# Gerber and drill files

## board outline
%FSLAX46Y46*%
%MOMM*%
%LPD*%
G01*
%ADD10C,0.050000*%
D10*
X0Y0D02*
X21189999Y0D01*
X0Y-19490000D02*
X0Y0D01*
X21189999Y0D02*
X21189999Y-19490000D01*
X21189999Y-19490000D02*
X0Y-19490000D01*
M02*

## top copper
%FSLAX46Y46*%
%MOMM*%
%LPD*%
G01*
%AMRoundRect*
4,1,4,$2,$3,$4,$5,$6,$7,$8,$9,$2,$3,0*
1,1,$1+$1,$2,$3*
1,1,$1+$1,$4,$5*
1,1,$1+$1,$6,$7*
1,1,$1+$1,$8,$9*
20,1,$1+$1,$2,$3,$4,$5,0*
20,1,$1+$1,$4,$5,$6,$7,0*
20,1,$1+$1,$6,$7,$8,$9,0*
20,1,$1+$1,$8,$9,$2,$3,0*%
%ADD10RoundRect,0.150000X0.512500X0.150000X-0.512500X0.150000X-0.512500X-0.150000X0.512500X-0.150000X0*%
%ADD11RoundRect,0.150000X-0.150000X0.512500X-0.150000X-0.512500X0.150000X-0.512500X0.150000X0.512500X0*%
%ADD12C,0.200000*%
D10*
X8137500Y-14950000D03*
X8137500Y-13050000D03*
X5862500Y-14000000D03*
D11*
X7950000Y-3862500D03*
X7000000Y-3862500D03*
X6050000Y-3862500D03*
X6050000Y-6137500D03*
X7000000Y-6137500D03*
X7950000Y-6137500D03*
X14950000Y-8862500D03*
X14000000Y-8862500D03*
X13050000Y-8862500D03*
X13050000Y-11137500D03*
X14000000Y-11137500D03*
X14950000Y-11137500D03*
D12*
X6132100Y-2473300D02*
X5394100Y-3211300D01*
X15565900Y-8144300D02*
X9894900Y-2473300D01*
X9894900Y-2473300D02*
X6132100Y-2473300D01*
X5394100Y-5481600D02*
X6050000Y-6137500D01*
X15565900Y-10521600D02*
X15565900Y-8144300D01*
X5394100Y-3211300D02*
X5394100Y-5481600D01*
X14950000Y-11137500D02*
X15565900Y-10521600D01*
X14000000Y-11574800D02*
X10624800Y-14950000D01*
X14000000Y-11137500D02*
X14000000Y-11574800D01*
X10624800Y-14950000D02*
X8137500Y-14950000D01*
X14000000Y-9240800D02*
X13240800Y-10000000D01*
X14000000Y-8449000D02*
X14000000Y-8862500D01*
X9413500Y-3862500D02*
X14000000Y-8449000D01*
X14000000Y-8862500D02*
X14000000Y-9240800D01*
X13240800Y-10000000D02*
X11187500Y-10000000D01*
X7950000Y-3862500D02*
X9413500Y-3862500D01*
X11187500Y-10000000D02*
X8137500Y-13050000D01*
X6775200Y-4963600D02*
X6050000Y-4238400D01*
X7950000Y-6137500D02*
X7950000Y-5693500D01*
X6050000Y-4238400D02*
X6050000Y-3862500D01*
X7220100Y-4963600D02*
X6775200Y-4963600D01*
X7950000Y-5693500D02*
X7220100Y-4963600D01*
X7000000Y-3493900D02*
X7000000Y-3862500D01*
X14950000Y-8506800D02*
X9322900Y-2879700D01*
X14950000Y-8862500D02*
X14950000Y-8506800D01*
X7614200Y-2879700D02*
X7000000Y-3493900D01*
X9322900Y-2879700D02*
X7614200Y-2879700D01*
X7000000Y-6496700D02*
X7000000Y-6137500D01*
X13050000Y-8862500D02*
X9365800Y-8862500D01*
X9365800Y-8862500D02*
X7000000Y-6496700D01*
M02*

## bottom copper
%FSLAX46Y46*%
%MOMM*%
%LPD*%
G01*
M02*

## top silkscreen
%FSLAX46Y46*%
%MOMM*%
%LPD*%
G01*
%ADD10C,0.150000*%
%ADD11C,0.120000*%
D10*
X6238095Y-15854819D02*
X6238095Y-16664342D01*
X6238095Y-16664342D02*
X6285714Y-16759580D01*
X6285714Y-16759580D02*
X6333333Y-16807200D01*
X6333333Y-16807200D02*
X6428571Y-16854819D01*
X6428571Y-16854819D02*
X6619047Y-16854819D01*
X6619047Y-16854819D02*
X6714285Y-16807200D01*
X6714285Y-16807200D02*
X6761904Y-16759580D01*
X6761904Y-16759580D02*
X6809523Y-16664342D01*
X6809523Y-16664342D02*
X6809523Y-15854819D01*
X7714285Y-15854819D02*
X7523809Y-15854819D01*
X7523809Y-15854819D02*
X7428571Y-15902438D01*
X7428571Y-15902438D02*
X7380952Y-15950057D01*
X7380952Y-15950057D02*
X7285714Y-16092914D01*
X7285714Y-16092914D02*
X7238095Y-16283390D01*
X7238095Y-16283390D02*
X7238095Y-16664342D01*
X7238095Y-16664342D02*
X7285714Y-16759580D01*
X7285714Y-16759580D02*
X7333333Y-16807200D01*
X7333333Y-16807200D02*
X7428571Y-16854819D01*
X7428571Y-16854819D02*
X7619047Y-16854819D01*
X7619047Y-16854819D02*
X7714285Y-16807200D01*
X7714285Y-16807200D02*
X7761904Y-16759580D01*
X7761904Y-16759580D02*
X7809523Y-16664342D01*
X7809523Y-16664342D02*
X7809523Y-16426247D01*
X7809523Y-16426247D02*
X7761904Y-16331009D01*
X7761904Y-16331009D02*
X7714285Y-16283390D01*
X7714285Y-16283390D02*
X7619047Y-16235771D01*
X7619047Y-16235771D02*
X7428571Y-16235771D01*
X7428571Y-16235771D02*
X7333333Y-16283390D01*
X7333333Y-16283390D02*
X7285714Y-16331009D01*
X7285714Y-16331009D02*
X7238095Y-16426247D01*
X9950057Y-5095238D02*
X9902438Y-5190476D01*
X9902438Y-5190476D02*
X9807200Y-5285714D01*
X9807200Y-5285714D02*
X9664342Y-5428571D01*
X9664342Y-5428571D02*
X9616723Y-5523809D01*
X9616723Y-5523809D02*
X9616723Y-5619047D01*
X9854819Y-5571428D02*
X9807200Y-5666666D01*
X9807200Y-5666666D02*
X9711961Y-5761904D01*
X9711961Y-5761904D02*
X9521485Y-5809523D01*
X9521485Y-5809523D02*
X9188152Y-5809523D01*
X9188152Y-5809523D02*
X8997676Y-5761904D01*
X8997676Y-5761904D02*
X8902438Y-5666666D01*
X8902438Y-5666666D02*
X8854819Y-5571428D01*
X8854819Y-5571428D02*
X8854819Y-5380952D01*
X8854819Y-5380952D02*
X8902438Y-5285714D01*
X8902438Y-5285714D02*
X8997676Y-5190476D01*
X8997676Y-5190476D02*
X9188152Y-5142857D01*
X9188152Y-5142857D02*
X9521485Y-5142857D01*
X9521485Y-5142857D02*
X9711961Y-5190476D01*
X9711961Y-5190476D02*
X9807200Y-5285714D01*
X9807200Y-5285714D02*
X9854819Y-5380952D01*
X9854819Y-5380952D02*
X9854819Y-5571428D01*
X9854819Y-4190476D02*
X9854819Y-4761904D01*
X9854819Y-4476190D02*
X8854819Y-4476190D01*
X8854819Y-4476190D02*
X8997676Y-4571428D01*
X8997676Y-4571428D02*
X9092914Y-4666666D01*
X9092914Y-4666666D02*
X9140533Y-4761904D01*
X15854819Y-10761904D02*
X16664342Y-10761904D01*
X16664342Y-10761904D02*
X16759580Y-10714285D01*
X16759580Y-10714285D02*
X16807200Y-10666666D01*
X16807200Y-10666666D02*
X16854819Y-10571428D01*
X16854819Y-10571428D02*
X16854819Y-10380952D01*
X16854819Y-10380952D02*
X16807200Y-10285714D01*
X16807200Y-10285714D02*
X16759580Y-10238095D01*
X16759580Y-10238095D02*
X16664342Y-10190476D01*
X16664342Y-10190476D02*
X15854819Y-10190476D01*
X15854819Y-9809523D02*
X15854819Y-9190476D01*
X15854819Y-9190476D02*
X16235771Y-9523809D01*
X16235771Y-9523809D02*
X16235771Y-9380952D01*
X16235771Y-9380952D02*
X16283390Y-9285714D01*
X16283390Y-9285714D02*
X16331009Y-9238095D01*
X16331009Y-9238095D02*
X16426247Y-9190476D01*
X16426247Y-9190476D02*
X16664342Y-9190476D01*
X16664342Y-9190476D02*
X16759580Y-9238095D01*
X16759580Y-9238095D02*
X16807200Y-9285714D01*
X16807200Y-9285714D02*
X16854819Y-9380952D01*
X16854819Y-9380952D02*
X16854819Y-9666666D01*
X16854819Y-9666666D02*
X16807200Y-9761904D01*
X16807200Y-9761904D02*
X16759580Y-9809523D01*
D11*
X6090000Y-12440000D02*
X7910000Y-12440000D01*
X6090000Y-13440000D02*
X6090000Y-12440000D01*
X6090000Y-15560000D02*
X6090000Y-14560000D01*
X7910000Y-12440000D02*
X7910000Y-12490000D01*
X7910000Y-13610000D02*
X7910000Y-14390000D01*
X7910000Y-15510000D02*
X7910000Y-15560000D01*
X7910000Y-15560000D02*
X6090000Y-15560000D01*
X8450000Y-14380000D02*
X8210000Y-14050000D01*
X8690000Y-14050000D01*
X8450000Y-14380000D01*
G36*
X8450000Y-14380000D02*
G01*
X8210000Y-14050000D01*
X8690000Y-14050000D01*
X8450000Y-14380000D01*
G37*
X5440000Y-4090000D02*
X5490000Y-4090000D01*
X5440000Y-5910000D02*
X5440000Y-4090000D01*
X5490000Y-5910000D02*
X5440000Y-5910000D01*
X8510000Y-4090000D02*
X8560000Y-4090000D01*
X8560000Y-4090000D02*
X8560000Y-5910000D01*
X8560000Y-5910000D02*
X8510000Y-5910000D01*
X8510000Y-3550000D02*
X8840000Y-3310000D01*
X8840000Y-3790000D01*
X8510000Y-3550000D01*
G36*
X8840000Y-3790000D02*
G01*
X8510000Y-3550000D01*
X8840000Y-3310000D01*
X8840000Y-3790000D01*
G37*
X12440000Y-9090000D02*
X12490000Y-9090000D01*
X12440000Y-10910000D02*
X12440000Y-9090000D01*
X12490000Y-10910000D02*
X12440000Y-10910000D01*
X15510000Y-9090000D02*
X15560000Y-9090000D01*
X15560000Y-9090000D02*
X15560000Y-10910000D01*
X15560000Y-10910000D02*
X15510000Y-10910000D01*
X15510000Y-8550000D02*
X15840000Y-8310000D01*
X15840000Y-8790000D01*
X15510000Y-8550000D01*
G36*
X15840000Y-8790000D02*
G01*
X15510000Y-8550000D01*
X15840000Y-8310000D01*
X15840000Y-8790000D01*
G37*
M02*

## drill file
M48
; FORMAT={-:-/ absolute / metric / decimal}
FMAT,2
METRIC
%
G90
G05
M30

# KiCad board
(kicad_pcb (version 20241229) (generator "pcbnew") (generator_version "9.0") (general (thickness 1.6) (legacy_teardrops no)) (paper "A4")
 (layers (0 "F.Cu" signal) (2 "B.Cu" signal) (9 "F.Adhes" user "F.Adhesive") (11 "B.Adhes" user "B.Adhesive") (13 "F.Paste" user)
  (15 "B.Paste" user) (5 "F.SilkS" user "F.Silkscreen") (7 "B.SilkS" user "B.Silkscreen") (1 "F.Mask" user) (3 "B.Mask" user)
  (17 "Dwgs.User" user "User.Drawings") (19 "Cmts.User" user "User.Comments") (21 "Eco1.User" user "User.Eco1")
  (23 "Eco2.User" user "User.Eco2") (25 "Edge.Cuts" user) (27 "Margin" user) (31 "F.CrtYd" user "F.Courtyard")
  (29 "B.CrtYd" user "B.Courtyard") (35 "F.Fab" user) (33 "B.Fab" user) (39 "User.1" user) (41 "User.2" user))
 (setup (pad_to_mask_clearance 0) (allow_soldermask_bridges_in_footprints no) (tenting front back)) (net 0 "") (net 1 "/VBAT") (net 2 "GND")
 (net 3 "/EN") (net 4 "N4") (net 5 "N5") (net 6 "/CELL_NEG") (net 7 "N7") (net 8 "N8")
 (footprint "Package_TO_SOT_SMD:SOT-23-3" (layer "F.Cu") (at 7 14 180)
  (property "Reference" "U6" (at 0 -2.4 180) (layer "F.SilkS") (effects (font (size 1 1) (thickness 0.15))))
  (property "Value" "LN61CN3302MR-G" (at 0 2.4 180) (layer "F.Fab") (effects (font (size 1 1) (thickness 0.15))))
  (fp_line (start 0.91 1.56) (end -0.91 1.56) (stroke (width 0.12) (type solid)) (layer "F.SilkS"))
  (fp_line (start 0.91 0.56) (end 0.91 1.56) (stroke (width 0.12) (type solid)) (layer "F.SilkS"))
  (fp_line (start 0.91 -1.56) (end 0.91 -0.56) (stroke (width 0.12) (type solid)) (layer "F.SilkS"))
  (fp_line (start -0.91 1.56) (end -0.91 1.51) (stroke (width 0.12) (type solid)) (layer "F.SilkS"))
  (fp_line (start -0.91 0.39) (end -0.91 -0.39) (stroke (width 0.12) (type solid)) (layer "F.SilkS"))
  (fp_line (start -0.91 -1.51) (end -0.91 -1.56) (stroke (width 0.12) (type solid)) (layer "F.SilkS"))
  (fp_line (start -0.91 -1.56) (end 0.91 -1.56) (stroke (width 0.12) (type solid)) (layer "F.SilkS"))
  (fp_poly (pts (xy -1.45 -0.38) (xy -1.21 -0.05) (xy -1.69 -0.05)) (stroke (width 0.12) (type solid)) (fill yes) (layer "F.SilkS"))
  (pad "1" smd roundrect (at -1.1375 -0.95 180) (size 1.325 0.6) (layers "F.Cu" "F.Mask" "F.Paste") (roundrect_rratio 0.25) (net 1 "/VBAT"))
  (pad "2" smd roundrect (at -1.1375 0.95 180) (size 1.325 0.6) (layers "F.Cu" "F.Mask" "F.Paste") (roundrect_rratio 0.25) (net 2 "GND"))
  (pad "3" smd roundrect (at 1.1375 0 180) (size 1.325 0.6) (layers "F.Cu" "F.Mask" "F.Paste") (roundrect_rratio 0.25) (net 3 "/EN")))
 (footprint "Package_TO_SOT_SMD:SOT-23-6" (layer "F.Cu") (at 7 5 -90)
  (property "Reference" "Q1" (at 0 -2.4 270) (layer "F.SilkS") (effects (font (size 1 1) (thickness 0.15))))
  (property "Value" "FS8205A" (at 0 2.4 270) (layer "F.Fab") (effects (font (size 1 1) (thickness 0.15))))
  (fp_line (start -0.91 1.56) (end -0.91 1.51) (stroke (width 0.12) (type solid)) (layer "F.SilkS"))
  (fp_line (start 0.91 1.56) (end -0.91 1.56) (stroke (width 0.12) (type solid)) (layer "F.SilkS"))
  (fp_line (start 0.91 1.51) (end 0.91 1.56) (stroke (width 0.12) (type solid)) (layer "F.SilkS"))
  (fp_line (start -0.91 -1.51) (end -0.91 -1.56) (stroke (width 0.12) (type solid)) (layer "F.SilkS"))
  (fp_line (start -0.91 -1.56) (end 0.91 -1.56) (stroke (width 0.12) (type solid)) (layer "F.SilkS"))
  (fp_line (start 0.91 -1.56) (end 0.91 -1.51) (stroke (width 0.12) (type solid)) (layer "F.SilkS"))
  (fp_poly (pts (xy -1.45 -1.51) (xy -1.69 -1.84) (xy -1.21 -1.84)) (stroke (width 0.12) (type solid)) (fill yes) (layer "F.SilkS"))
  (pad "1" smd roundrect (at -1.1375 -0.95 270) (size 1.325 0.6) (layers "F.Cu" "F.Mask" "F.Paste") (roundrect_rratio 0.25) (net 2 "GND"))
  (pad "2" smd roundrect (at -1.1375 0 270) (size 1.325 0.6) (layers "F.Cu" "F.Mask" "F.Paste") (roundrect_rratio 0.25) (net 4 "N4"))
  (pad "3" smd roundrect (at -1.1375 0.95 270) (size 1.325 0.6) (layers "F.Cu" "F.Mask" "F.Paste") (roundrect_rratio 0.25) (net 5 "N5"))
  (pad "4" smd roundrect (at 1.1375 0.95 270) (size 1.325 0.6) (layers "F.Cu" "F.Mask" "F.Paste") (roundrect_rratio 0.25)
   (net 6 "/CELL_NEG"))
  (pad "5" smd roundrect (at 1.1375 0 270) (size 1.325 0.6) (layers "F.Cu" "F.Mask" "F.Paste") (roundrect_rratio 0.25) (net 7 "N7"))
  (pad "6" smd roundrect (at 1.1375 -0.95 270) (size 1.325 0.6) (layers "F.Cu" "F.Mask" "F.Paste") (roundrect_rratio 0.25) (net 5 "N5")))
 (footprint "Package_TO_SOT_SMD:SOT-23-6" (layer "F.Cu") (at 14 10 -90)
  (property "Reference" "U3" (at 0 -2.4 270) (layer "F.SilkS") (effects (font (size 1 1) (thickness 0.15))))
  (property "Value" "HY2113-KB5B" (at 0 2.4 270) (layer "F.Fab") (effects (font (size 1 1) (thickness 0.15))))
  (fp_line (start -0.91 1.56) (end -0.91 1.51) (stroke (width 0.12) (type solid)) (layer "F.SilkS"))
  (fp_line (start 0.91 1.56) (end -0.91 1.56) (stroke (width 0.12) (type solid)) (layer "F.SilkS"))
  (fp_line (start 0.91 1.51) (end 0.91 1.56) (stroke (width 0.12) (type solid)) (layer "F.SilkS"))
  (fp_line (start -0.91 -1.51) (end -0.91 -1.56) (stroke (width 0.12) (type solid)) (layer "F.SilkS"))
  (fp_line (start -0.91 -1.56) (end 0.91 -1.56) (stroke (width 0.12) (type solid)) (layer "F.SilkS"))
  (fp_line (start 0.91 -1.56) (end 0.91 -1.51) (stroke (width 0.12) (type solid)) (layer "F.SilkS"))
  (fp_poly (pts (xy -1.45 -1.51) (xy -1.69 -1.84) (xy -1.21 -1.84)) (stroke (width 0.12) (type solid)) (fill yes) (layer "F.SilkS"))
  (pad "1" smd roundrect (at -1.1375 -0.95 270) (size 1.325 0.6) (layers "F.Cu" "F.Mask" "F.Paste") (roundrect_rratio 0.25) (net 4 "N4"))
  (pad "2" smd roundrect (at -1.1375 0 270) (size 1.325 0.6) (layers "F.Cu" "F.Mask" "F.Paste") (roundrect_rratio 0.25) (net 2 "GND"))
  (pad "3" smd roundrect (at -1.1375 0.95 270) (size 1.325 0.6) (layers "F.Cu" "F.Mask" "F.Paste") (roundrect_rratio 0.25) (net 7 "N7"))
  (pad "4" smd roundrect (at 1.1375 0.95 270) (size 1.325 0.6) (layers "F.Cu" "F.Mask" "F.Paste") (roundrect_rratio 0.25) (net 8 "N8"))
  (pad "5" smd roundrect (at 1.1375 0 270) (size 1.325 0.6) (layers "F.Cu" "F.Mask" "F.Paste") (roundrect_rratio 0.25) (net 1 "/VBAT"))
  (pad "6" smd roundrect (at 1.1375 -0.95 270) (size 1.325 0.6) (layers "F.Cu" "F.Mask" "F.Paste") (roundrect_rratio 0.25)
   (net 6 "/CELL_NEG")))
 (gr_line (start 0 0) (end 21.189999 0) (stroke (width 0.05) (type default)) (layer "Edge.Cuts"))
 (gr_line (start 0 19.49) (end 0 0) (stroke (width 0.05) (type default)) (layer "Edge.Cuts"))
 (gr_line (start 21.189999 0) (end 21.189999 19.49) (stroke (width 0.05) (type default)) (layer "Edge.Cuts"))
 (gr_line (start 21.189999 19.49) (end 0 19.49) (stroke (width 0.05) (type default)) (layer "Edge.Cuts"))
 (segment (start 6.1321 2.4733) (end 5.3941 3.2113) (width 0.2) (layer "F.Cu") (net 6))
 (segment (start 15.5659 8.1443) (end 9.8949 2.4733) (width 0.2) (layer "F.Cu") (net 6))
 (segment (start 9.8949 2.4733) (end 6.1321 2.4733) (width 0.2) (layer "F.Cu") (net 6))
 (segment (start 5.3941 5.4816) (end 6.05 6.1375) (width 0.2) (layer "F.Cu") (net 6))
 (segment (start 15.5659 10.5216) (end 15.5659 8.1443) (width 0.2) (layer "F.Cu") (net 6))
 (segment (start 5.3941 3.2113) (end 5.3941 5.4816) (width 0.2) (layer "F.Cu") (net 6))
 (segment (start 14.95 11.1375) (end 15.5659 10.5216) (width 0.2) (layer "F.Cu") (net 6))
 (segment (start 14 11.5748) (end 10.6248 14.95) (width 0.2) (layer "F.Cu") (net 1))
 (segment (start 14 11.1375) (end 14 11.5748) (width 0.2) (layer "F.Cu") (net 1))
 (segment (start 10.6248 14.95) (end 8.1375 14.95) (width 0.2) (layer "F.Cu") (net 1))
 (segment (start 14 9.2408) (end 13.2408 10) (width 0.2) (layer "F.Cu") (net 2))
 (segment (start 14 8.449) (end 14 8.8625) (width 0.2) (layer "F.Cu") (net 2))
 (segment (start 9.4135 3.8625) (end 14 8.449) (width 0.2) (layer "F.Cu") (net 2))
 (segment (start 14 8.8625) (end 14 9.2408) (width 0.2) (layer "F.Cu") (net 2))
 (segment (start 13.2408 10) (end 11.1875 10) (width 0.2) (layer "F.Cu") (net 2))
 (segment (start 7.95 3.8625) (end 9.4135 3.8625) (width 0.2) (layer "F.Cu") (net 2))
 (segment (start 11.1875 10) (end 8.1375 13.05) (width 0.2) (layer "F.Cu") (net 2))
 (segment (start 6.7752 4.9636) (end 6.05 4.2384) (width 0.2) (layer "F.Cu") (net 5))
 (segment (start 7.95 6.1375) (end 7.95 5.6935) (width 0.2) (layer "F.Cu") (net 5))
 (segment (start 6.05 4.2384) (end 6.05 3.8625) (width 0.2) (layer "F.Cu") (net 5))
 (segment (start 7.2201 4.9636) (end 6.7752 4.9636) (width 0.2) (layer "F.Cu") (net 5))
 (segment (start 7.95 5.6935) (end 7.2201 4.9636) (width 0.2) (layer "F.Cu") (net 5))
 (segment (start 7 3.4939) (end 7 3.8625) (width 0.2) (layer "F.Cu") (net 4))
 (segment (start 14.95 8.5068) (end 9.3229 2.8797) (width 0.2) (layer "F.Cu") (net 4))
 (segment (start 14.95 8.8625) (end 14.95 8.5068) (width 0.2) (layer "F.Cu") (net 4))
 (segment (start 7.6142 2.8797) (end 7 3.4939) (width 0.2) (layer "F.Cu") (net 4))
 (segment (start 9.3229 2.8797) (end 7.6142 2.8797) (width 0.2) (layer "F.Cu") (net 4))
 (segment (start 7 6.4967) (end 7 6.1375) (width 0.2) (layer "F.Cu") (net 7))
 (segment (start 13.05 8.8625) (end 9.3658 8.8625) (width 0.2) (layer "F.Cu") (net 7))
 (segment (start 9.3658 8.8625) (end 7 6.4967) (width 0.2) (layer "F.Cu") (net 7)))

